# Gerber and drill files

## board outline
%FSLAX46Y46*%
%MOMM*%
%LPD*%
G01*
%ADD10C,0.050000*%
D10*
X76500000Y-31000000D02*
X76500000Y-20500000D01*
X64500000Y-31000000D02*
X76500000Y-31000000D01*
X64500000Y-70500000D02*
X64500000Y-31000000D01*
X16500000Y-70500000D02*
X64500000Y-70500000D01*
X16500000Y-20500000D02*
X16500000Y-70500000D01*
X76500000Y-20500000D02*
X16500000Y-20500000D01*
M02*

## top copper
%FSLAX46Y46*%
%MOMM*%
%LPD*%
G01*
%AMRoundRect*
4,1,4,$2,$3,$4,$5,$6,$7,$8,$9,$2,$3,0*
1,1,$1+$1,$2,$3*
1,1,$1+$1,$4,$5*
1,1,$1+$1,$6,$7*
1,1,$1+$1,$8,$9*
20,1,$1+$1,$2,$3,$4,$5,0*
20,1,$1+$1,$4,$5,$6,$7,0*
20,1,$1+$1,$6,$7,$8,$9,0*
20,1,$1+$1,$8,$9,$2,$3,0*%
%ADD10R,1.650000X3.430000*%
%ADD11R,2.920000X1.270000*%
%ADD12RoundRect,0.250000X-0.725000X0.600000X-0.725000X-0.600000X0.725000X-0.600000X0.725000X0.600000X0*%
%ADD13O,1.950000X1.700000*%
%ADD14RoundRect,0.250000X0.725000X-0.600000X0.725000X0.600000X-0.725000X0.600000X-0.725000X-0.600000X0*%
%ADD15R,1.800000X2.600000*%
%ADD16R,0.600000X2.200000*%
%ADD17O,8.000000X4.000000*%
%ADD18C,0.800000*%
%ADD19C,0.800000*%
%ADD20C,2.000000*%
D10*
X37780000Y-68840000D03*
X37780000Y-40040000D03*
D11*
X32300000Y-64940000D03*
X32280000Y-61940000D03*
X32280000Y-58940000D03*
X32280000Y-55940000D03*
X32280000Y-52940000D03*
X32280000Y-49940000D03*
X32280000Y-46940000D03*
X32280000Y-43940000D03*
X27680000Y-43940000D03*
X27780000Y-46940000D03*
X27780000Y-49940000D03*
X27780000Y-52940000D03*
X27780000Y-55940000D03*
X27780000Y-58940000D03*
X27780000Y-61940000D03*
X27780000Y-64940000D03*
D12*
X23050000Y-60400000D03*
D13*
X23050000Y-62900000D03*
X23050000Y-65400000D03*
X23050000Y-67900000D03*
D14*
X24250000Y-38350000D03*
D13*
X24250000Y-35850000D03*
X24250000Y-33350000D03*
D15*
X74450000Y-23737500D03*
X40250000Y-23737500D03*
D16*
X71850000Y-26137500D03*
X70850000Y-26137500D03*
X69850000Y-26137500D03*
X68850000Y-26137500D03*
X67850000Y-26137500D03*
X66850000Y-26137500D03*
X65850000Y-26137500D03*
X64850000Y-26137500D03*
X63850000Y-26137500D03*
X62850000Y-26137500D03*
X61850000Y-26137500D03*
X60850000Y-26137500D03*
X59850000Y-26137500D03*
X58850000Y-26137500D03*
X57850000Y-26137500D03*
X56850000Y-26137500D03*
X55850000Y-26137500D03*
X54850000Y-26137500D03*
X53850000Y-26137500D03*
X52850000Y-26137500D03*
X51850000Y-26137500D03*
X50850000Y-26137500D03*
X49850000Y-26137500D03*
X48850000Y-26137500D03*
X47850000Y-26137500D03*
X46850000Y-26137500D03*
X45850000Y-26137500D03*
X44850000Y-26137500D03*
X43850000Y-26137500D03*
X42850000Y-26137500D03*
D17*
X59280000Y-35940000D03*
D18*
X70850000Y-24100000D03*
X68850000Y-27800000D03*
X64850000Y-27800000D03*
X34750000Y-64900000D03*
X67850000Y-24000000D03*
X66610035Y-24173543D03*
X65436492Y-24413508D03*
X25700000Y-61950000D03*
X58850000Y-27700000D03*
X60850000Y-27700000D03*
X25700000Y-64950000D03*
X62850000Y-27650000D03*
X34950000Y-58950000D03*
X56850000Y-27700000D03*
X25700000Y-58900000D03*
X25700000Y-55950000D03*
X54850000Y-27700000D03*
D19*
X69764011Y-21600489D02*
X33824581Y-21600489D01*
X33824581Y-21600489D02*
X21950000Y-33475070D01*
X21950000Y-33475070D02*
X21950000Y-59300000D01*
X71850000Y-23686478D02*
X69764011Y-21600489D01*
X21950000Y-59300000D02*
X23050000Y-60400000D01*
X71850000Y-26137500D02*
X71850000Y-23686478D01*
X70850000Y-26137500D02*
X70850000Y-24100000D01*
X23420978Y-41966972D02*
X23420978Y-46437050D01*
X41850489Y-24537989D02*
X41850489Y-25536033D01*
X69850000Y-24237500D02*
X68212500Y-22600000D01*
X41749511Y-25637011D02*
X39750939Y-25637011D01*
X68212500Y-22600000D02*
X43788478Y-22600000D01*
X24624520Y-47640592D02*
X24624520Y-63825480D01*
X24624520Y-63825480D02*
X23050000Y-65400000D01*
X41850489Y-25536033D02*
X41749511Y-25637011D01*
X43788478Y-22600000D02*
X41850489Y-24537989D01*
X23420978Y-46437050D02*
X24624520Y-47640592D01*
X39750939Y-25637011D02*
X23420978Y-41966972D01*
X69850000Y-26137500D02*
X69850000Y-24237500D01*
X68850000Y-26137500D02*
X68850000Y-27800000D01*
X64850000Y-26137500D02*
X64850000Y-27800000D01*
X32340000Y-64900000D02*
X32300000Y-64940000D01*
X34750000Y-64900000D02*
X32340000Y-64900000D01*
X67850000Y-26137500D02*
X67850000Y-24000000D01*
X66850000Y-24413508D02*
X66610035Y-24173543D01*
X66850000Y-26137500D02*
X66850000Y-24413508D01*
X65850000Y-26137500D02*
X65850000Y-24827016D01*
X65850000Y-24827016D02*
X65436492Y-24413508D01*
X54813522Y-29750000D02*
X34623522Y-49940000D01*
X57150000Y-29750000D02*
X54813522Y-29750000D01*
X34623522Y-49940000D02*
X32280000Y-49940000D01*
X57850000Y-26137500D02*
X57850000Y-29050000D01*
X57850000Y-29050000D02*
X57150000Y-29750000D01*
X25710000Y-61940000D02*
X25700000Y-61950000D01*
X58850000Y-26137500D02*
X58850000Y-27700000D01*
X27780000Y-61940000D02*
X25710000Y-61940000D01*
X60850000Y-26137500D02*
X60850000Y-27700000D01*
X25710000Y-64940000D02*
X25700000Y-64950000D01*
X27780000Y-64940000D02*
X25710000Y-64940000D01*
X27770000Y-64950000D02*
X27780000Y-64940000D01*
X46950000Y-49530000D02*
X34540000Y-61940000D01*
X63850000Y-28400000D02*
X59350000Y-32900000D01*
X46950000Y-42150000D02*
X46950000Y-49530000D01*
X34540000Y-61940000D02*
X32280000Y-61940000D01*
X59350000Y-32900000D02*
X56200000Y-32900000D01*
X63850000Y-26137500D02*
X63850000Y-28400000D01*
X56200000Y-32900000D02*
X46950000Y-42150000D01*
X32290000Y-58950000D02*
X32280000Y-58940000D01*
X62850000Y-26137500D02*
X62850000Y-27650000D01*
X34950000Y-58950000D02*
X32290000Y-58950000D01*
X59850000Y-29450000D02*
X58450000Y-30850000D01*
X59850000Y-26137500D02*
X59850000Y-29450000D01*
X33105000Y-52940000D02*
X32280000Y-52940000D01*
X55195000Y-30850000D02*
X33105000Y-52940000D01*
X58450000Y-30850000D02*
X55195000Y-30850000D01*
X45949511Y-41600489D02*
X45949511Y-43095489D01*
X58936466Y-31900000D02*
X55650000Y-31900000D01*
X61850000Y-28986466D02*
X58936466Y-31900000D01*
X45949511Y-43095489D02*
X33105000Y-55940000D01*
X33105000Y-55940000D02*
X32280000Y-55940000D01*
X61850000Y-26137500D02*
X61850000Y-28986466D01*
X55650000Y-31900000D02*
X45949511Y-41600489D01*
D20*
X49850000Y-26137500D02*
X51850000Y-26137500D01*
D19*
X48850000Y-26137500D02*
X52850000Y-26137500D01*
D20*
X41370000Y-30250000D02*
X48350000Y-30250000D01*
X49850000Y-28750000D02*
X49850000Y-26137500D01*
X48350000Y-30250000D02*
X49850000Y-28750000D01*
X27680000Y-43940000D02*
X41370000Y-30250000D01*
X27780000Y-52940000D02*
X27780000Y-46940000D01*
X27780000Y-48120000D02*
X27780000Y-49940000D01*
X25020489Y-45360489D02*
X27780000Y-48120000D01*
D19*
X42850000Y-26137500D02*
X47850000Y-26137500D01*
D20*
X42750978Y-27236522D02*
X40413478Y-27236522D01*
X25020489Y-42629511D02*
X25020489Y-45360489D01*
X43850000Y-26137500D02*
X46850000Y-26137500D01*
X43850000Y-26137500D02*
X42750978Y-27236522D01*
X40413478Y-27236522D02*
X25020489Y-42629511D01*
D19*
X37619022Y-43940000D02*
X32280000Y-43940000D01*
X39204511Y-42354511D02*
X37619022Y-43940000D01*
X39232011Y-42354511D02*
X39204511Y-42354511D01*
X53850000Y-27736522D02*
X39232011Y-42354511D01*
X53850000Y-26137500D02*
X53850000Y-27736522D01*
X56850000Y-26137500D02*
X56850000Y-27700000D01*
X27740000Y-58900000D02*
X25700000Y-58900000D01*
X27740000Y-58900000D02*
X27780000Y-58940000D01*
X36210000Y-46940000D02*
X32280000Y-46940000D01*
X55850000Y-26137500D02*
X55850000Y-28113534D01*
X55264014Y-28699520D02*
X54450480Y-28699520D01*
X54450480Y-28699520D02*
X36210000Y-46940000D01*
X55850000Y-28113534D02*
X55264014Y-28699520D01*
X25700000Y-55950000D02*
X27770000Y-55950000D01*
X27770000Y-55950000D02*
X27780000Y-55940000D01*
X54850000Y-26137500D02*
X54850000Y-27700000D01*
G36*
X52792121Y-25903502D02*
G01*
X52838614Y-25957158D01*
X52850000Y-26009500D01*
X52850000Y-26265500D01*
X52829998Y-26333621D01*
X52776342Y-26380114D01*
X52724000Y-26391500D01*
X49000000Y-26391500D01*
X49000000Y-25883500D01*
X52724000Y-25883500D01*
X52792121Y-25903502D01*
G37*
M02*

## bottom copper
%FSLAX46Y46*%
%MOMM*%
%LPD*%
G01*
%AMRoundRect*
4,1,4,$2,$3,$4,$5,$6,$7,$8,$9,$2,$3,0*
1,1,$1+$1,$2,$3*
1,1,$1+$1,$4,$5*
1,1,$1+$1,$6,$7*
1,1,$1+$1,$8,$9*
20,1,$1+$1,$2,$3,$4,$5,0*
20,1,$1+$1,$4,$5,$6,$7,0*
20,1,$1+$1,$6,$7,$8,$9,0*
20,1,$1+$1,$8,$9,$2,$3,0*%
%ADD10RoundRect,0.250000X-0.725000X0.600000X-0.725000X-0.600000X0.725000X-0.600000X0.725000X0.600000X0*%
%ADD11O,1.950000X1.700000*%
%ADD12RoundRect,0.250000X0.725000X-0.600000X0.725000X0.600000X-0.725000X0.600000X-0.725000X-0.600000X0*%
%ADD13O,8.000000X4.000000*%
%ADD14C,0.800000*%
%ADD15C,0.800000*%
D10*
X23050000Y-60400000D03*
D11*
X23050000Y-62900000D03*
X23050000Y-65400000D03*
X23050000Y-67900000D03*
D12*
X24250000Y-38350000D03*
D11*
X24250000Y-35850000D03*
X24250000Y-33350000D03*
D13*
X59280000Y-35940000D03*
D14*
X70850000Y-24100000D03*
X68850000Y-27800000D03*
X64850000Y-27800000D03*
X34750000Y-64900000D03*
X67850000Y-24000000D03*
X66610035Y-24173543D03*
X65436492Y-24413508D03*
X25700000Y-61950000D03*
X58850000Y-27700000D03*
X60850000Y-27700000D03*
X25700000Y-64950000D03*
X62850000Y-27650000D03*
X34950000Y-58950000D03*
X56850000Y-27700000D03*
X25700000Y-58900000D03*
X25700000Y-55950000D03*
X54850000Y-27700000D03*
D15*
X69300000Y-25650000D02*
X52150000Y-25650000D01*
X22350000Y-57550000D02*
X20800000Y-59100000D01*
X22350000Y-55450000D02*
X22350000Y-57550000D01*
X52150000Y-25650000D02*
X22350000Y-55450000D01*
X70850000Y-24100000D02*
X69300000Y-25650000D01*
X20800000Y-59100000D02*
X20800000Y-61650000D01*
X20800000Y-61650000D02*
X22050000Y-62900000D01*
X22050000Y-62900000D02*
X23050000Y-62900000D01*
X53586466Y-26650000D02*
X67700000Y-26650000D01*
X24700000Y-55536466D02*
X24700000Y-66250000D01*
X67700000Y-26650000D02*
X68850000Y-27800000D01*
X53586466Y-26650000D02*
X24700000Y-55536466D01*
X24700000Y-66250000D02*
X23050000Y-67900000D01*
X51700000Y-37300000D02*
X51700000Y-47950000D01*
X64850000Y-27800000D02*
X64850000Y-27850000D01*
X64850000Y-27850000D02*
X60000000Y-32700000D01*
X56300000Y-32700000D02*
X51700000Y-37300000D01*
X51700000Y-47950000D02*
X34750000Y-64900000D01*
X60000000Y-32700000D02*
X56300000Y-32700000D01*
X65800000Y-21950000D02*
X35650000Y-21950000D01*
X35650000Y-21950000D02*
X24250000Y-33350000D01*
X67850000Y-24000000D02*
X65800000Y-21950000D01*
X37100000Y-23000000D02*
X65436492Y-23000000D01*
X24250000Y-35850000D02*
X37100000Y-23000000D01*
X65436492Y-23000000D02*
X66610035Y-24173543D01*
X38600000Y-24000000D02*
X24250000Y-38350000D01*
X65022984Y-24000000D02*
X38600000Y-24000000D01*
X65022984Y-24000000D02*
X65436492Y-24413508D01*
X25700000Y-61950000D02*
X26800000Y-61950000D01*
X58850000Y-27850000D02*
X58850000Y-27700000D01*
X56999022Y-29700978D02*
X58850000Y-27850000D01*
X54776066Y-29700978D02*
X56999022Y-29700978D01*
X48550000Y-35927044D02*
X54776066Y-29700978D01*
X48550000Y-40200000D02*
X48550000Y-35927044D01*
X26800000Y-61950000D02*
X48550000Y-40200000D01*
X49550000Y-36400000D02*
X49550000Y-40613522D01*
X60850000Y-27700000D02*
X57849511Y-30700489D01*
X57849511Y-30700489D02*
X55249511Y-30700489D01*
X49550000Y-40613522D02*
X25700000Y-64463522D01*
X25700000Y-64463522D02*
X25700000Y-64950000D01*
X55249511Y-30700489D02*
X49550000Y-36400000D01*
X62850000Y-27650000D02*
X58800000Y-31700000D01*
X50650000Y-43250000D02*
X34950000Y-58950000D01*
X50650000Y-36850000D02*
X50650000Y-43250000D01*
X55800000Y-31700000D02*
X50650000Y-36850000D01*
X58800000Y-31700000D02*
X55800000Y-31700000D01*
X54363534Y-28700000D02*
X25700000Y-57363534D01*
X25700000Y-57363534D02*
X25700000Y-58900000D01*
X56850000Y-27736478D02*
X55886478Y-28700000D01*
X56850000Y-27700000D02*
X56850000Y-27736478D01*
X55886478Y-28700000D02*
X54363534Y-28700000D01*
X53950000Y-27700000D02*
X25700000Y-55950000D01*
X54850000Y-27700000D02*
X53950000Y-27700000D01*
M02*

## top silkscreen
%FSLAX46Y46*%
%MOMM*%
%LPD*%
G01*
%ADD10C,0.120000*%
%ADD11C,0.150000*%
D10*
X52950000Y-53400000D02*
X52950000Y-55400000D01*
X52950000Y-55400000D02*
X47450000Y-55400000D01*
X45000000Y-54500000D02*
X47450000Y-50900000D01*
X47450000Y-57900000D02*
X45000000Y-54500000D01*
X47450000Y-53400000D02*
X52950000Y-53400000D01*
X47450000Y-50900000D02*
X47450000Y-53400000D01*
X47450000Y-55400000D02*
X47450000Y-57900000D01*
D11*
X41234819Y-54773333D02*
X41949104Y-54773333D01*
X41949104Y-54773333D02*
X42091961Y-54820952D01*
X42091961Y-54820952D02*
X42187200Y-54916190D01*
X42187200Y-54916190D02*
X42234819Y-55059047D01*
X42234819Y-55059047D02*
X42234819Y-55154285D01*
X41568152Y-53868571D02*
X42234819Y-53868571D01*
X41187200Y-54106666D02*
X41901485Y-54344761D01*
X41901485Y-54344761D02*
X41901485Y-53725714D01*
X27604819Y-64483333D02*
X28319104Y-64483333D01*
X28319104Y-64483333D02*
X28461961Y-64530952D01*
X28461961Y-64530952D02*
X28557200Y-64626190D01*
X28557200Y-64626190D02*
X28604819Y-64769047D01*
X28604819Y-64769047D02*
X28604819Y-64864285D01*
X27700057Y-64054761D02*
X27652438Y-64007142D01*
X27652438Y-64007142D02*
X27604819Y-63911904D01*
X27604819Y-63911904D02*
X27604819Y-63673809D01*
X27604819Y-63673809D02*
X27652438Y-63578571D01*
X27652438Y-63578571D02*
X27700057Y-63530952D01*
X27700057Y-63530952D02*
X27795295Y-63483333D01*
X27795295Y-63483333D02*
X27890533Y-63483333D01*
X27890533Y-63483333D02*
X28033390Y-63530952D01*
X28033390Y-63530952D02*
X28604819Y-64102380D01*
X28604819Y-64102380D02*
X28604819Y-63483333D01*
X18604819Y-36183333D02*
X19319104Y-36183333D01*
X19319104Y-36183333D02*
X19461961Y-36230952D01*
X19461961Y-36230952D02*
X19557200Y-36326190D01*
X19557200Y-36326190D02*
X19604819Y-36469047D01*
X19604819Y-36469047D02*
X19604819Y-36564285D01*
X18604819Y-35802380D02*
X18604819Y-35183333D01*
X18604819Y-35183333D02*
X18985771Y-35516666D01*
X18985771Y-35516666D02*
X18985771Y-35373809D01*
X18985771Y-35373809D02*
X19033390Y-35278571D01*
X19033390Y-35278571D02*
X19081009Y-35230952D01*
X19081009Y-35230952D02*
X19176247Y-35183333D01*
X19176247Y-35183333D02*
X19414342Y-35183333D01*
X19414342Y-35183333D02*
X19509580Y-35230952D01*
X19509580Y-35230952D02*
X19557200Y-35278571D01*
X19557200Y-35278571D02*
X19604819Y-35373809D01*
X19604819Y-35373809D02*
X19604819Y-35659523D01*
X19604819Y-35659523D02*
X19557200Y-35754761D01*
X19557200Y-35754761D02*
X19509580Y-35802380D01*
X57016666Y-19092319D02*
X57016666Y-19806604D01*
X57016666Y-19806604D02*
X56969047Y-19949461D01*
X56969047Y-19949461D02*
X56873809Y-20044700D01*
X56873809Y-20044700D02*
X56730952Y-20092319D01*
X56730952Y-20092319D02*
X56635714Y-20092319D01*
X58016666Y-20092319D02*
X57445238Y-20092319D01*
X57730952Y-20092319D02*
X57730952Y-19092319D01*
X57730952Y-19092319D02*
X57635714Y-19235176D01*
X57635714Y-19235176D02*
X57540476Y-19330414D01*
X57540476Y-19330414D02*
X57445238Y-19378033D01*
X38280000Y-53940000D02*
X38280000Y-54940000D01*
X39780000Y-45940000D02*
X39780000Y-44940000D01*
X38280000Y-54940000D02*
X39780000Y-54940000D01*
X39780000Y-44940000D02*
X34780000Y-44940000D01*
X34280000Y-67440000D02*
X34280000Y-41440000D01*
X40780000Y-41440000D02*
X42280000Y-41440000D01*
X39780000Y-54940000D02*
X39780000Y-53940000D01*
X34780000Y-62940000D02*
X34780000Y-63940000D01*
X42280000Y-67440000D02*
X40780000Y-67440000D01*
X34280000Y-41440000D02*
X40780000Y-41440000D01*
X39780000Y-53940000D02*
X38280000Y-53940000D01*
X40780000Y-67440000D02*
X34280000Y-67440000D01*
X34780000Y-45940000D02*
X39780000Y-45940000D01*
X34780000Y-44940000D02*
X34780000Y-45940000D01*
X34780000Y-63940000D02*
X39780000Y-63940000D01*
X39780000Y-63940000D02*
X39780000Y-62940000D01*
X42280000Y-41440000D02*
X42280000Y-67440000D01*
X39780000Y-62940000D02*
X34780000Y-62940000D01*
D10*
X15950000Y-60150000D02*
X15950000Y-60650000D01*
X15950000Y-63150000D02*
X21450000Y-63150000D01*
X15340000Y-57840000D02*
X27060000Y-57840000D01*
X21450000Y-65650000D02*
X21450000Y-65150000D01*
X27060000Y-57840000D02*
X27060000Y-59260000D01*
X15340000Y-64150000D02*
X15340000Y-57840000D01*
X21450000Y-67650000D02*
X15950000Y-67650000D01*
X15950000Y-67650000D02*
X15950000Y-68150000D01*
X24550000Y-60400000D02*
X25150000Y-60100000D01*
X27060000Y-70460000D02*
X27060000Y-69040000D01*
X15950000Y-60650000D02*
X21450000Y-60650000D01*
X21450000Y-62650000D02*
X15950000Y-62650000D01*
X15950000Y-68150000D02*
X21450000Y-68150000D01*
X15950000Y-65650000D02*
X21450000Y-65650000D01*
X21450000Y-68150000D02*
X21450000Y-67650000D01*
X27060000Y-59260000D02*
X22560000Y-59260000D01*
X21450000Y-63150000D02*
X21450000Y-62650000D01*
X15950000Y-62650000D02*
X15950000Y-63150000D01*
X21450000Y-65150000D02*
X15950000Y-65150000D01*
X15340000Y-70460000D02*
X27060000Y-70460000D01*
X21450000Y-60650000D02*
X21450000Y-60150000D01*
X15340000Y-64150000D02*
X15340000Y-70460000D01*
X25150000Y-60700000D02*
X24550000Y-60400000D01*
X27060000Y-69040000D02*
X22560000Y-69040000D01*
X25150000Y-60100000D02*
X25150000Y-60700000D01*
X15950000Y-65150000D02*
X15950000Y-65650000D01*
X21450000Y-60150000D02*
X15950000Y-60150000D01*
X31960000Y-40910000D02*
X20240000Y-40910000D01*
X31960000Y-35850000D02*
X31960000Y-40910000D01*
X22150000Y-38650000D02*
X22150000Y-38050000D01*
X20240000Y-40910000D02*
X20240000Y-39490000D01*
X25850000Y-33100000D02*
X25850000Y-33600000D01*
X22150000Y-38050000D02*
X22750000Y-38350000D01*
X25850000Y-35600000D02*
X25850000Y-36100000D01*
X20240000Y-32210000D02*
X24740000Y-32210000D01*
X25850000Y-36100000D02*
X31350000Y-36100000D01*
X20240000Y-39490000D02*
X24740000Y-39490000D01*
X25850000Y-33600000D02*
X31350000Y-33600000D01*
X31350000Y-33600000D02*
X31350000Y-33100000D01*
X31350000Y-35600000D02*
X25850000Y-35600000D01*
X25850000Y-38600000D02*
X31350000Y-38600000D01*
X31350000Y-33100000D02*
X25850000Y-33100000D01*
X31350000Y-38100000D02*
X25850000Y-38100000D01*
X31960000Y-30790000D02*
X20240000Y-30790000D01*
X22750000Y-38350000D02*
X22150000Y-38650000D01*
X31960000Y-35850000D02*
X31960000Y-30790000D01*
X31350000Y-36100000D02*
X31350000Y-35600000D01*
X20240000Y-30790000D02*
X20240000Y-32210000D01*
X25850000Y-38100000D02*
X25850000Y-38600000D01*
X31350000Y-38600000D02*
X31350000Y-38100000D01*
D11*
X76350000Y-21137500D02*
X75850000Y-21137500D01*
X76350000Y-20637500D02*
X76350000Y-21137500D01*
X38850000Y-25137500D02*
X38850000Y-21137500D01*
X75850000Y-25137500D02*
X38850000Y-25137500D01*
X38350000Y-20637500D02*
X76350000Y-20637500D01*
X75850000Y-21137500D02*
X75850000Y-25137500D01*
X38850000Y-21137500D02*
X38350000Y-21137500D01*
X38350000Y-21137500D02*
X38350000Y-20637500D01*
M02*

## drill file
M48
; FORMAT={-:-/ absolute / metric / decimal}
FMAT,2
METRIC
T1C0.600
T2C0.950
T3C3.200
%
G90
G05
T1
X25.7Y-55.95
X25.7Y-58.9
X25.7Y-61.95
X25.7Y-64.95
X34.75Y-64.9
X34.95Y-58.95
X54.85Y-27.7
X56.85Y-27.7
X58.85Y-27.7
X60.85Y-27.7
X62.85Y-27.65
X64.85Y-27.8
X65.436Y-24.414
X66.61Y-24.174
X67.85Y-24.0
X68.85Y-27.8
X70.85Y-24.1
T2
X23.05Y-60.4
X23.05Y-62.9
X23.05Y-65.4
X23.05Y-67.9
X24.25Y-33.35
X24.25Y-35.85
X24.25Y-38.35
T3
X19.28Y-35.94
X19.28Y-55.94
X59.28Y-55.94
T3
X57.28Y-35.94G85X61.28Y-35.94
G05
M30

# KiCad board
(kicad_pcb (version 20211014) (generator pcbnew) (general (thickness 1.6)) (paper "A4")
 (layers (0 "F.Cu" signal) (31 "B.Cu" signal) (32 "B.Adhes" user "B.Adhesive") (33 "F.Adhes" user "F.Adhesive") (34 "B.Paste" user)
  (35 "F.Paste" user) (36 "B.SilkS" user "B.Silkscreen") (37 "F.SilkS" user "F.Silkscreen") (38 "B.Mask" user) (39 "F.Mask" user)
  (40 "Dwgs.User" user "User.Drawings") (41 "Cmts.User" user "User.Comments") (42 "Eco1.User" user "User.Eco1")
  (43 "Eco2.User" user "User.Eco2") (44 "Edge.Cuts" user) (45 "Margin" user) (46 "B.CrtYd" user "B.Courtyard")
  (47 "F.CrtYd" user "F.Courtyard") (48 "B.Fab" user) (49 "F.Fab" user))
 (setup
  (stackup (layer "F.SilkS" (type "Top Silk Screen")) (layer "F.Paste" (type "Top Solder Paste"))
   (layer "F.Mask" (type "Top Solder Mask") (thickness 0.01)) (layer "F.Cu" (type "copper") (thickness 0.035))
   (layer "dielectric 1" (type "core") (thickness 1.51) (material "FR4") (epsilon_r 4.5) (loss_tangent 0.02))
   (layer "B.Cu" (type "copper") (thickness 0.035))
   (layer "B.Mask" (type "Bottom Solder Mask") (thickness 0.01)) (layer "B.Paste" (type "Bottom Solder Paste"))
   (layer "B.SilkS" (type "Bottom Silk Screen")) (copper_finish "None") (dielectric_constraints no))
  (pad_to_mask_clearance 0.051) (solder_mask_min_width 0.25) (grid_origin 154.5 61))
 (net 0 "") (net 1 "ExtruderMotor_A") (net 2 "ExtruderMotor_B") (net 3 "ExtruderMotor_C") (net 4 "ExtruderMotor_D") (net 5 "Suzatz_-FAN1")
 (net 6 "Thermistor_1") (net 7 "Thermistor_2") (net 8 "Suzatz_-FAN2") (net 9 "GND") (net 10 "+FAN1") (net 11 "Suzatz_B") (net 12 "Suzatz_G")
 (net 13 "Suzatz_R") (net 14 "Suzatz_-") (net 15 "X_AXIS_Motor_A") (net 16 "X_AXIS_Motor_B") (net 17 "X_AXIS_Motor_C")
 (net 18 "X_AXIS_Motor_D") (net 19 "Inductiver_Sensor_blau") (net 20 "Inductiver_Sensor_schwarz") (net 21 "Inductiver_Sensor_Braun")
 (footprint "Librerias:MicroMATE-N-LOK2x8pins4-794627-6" (layer "F.Cu") (at 37.78 54.44 90)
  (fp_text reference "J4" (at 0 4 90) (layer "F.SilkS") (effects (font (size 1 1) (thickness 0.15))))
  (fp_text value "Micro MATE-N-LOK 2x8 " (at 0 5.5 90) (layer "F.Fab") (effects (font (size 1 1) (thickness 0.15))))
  (fp_line (start 0.5 0.5) (end -0.5 0.5) (layer "F.SilkS") (width 0.15))
  (fp_line (start 8.5 2) (end 9.5 2) (layer "F.SilkS") (width 0.15))
  (fp_line (start -0.5 0.5) (end -0.5 2) (layer "F.SilkS") (width 0.15))
  (fp_line (start 9.5 2) (end 9.5 -3) (layer "F.SilkS") (width 0.15))
  (fp_line (start -13 -3.5) (end 13 -3.5) (layer "F.SilkS") (width 0.15))
  (fp_line (start 13 3) (end 13 4.5) (layer "F.SilkS") (width 0.15))
  (fp_line (start -0.5 2) (end 0.5 2) (layer "F.SilkS") (width 0.15))
  (fp_line (start -8.5 -3) (end -9.5 -3) (layer "F.SilkS") (width 0.15))
  (fp_line (start -13 4.5) (end -13 3) (layer "F.SilkS") (width 0.15))
  (fp_line (start 13 -3.5) (end 13 3) (layer "F.SilkS") (width 0.15))
  (fp_line (start 0.5 2) (end 0.5 0.5) (layer "F.SilkS") (width 0.15))
  (fp_line (start -13 3) (end -13 -3.5) (layer "F.SilkS") (width 0.15))
  (fp_line (start 8.5 -3) (end 8.5 2) (layer "F.SilkS") (width 0.15))
  (fp_line (start 9.5 -3) (end 8.5 -3) (layer "F.SilkS") (width 0.15))
  (fp_line (start -9.5 -3) (end -9.5 2) (layer "F.SilkS") (width 0.15))
  (fp_line (start -9.5 2) (end -8.5 2) (layer "F.SilkS") (width 0.15))
  (fp_line (start 13 4.5) (end -13 4.5) (layer "F.SilkS") (width 0.15))
  (fp_line (start -8.5 2) (end -8.5 -3) (layer "F.SilkS") (width 0.15))
  (pad "0" smd rect locked (at -14.4 0 90) (size 3.43 1.65) (layers "F.Cu" "F.Paste" "F.Mask"))
  (pad "0" smd rect locked (at 14.4 0 90) (size 3.43 1.65) (layers "F.Cu" "F.Paste" "F.Mask"))
  (pad "1" smd rect locked (at -10.5 -5.48 270) (size 1.27 2.92) (layers "F.Cu" "F.Paste" "F.Mask") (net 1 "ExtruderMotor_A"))
  (pad "2" smd rect locked (at -7.5 -5.5 270) (size 1.27 2.92) (layers "F.Cu" "F.Paste" "F.Mask") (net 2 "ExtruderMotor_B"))
  (pad "3" smd rect locked (at -4.5 -5.5 270) (size 1.27 2.92) (layers "F.Cu" "F.Paste" "F.Mask") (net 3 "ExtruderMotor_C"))
  (pad "4" smd rect locked (at -1.5 -5.5 270) (size 1.27 2.92) (layers "F.Cu" "F.Paste" "F.Mask") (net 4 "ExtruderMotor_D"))
  (pad "5" smd rect locked (at 1.5 -5.5 270) (size 1.27 2.92) (layers "F.Cu" "F.Paste" "F.Mask") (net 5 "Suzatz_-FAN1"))
  (pad "6" smd rect locked (at 4.5 -5.5 270) (size 1.27 2.92) (layers "F.Cu" "F.Paste" "F.Mask") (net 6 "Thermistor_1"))
  (pad "7" smd rect locked (at 7.5 -5.5 270) (size 1.27 2.92) (layers "F.Cu" "F.Paste" "F.Mask") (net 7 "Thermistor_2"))
  (pad "8" smd rect locked (at 10.5 -5.5 270) (size 1.27 2.92) (layers "F.Cu" "F.Paste" "F.Mask") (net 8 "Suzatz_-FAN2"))
  (pad "9" smd rect locked (at 10.5 -10.1 270) (size 1.27 2.92) (layers "F.Cu" "F.Paste" "F.Mask") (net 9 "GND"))
  (pad "10" smd rect locked (at 7.5 -10 270) (size 1.27 2.92) (layers "F.Cu" "F.Paste" "F.Mask") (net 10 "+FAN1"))
  (pad "11" smd rect locked (at 4.5 -10 270) (size 1.27 2.92) (layers "F.Cu" "F.Paste" "F.Mask") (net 10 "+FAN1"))
  (pad "12" smd rect locked (at 1.5 -10 270) (size 1.27 2.92) (layers "F.Cu" "F.Paste" "F.Mask") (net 10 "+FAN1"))
  (pad "13" smd rect locked (at -1.5 -10 270) (size 1.27 2.92) (layers "F.Cu" "F.Paste" "F.Mask") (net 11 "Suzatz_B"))
  (pad "14" smd rect locked (at -4.5 -10 270) (size 1.27 2.92) (layers "F.Cu" "F.Paste" "F.Mask") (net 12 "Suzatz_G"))
  (pad "15" smd rect locked (at -7.5 -10 270) (size 1.27 2.92) (layers "F.Cu" "F.Paste" "F.Mask") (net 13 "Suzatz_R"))
  (pad "16" smd rect locked (at -10.5 -10 270) (size 1.27 2.92) (layers "F.Cu" "F.Paste" "F.Mask") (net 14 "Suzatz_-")))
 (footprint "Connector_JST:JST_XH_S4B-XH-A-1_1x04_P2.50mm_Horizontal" (layer "F.Cu") (at 23.05 60.4 -90)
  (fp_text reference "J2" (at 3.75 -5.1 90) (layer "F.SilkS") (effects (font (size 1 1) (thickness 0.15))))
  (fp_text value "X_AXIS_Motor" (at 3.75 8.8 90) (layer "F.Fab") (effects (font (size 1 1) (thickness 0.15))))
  (fp_line (start -0.25 7.1) (end 0.25 7.1) (layer "F.SilkS") (width 0.12))
  (fp_line (start 2.75 7.1) (end 2.75 1.6) (layer "F.SilkS") (width 0.12))
  (fp_line (start -2.56 7.71) (end -2.56 -4.01) (layer "F.SilkS") (width 0.12))
  (fp_line (start 5.25 1.6) (end 4.75 1.6) (layer "F.SilkS") (width 0.12))
  (fp_line (start -2.56 -4.01) (end -1.14 -4.01) (layer "F.SilkS") (width 0.12))
  (fp_line (start 3.75 7.71) (end -2.56 7.71) (layer "F.SilkS") (width 0.12))
  (fp_line (start 7.25 1.6) (end 7.25 7.1) (layer "F.SilkS") (width 0.12))
  (fp_line (start 7.25 7.1) (end 7.75 7.1) (layer "F.SilkS") (width 0.12))
  (fp_line (start 0 -1.5) (end -0.3 -2.1) (layer "F.SilkS") (width 0.12))
  (fp_line (start 10.06 -4.01) (end 8.64 -4.01) (layer "F.SilkS") (width 0.12))
  (fp_line (start 0.25 7.1) (end 0.25 1.6) (layer "F.SilkS") (width 0.12))
  (fp_line (start 2.25 1.6) (end 2.25 7.1) (layer "F.SilkS") (width 0.12))
  (fp_line (start 7.75 7.1) (end 7.75 1.6) (layer "F.SilkS") (width 0.12))
  (fp_line (start 5.25 7.1) (end 5.25 1.6) (layer "F.SilkS") (width 0.12))
  (fp_line (start 7.75 1.6) (end 7.25 1.6) (layer "F.SilkS") (width 0.12))
  (fp_line (start -1.14 -4.01) (end -1.14 0.49) (layer "F.SilkS") (width 0.12))
  (fp_line (start 2.75 1.6) (end 2.25 1.6) (layer "F.SilkS") (width 0.12))
  (fp_line (start 2.25 7.1) (end 2.75 7.1) (layer "F.SilkS") (width 0.12))
  (fp_line (start 4.75 1.6) (end 4.75 7.1) (layer "F.SilkS") (width 0.12))
  (fp_line (start 10.06 7.71) (end 10.06 -4.01) (layer "F.SilkS") (width 0.12))
  (fp_line (start 0.25 1.6) (end -0.25 1.6) (layer "F.SilkS") (width 0.12))
  (fp_line (start 3.75 7.71) (end 10.06 7.71) (layer "F.SilkS") (width 0.12))
  (fp_line (start 0.3 -2.1) (end 0 -1.5) (layer "F.SilkS") (width 0.12))
  (fp_line (start 8.64 -4.01) (end 8.64 0.49) (layer "F.SilkS") (width 0.12))
  (fp_line (start -0.3 -2.1) (end 0.3 -2.1) (layer "F.SilkS") (width 0.12))
  (fp_line (start 4.75 7.1) (end 5.25 7.1) (layer "F.SilkS") (width 0.12))
  (fp_line (start -0.25 1.6) (end -0.25 7.1) (layer "F.SilkS") (width 0.12))
  (pad "1" thru_hole roundrect locked (at 0 0 270) (size 1.7 1.95) (drill 0.95) (layers *.Cu *.Mask) (roundrect_rratio 0.147059)
   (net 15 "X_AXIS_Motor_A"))
  (pad "2" thru_hole oval locked (at 2.5 0 270) (size 1.7 1.95) (drill 0.95) (layers *.Cu *.Mask) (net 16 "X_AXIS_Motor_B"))
  (pad "3" thru_hole oval locked (at 5 0 270) (size 1.7 1.95) (drill 0.95) (layers *.Cu *.Mask) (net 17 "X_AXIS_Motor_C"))
  (pad "4" thru_hole oval locked (at 7.5 0 270) (size 1.7 1.95) (drill 0.95) (layers *.Cu *.Mask) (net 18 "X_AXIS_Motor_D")))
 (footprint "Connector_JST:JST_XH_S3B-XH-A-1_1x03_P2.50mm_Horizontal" (layer "F.Cu") (at 24.25 38.35 90)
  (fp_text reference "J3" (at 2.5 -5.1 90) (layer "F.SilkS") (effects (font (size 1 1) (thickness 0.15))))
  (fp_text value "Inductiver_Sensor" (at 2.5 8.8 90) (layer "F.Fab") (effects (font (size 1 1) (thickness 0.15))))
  (fp_line (start -2.56 7.71) (end -2.56 -4.01) (layer "F.SilkS") (width 0.12))
  (fp_line (start 2.5 7.71) (end -2.56 7.71) (layer "F.SilkS") (width 0.12))
  (fp_line (start -0.3 -2.1) (end 0.3 -2.1) (layer "F.SilkS") (width 0.12))
  (fp_line (start -2.56 -4.01) (end -1.14 -4.01) (layer "F.SilkS") (width 0.12))
  (fp_line (start 5.25 1.6) (end 4.75 1.6) (layer "F.SilkS") (width 0.12))
  (fp_line (start 0.3 -2.1) (end 0 -1.5) (layer "F.SilkS") (width 0.12))
  (fp_line (start 2.75 1.6) (end 2.25 1.6) (layer "F.SilkS") (width 0.12))
  (fp_line (start 6.14 -4.01) (end 6.14 0.49) (layer "F.SilkS") (width 0.12))
  (fp_line (start 2.25 1.6) (end 2.25 7.1) (layer "F.SilkS") (width 0.12))
  (fp_line (start -1.14 -4.01) (end -1.14 0.49) (layer "F.SilkS") (width 0.12))
  (fp_line (start 4.75 1.6) (end 4.75 7.1) (layer "F.SilkS") (width 0.12))
  (fp_line (start 4.75 7.1) (end 5.25 7.1) (layer "F.SilkS") (width 0.12))
  (fp_line (start 2.75 7.1) (end 2.75 1.6) (layer "F.SilkS") (width 0.12))
  (fp_line (start -0.25 1.6) (end -0.25 7.1) (layer "F.SilkS") (width 0.12))
  (fp_line (start 5.25 7.1) (end 5.25 1.6) (layer "F.SilkS") (width 0.12))
  (fp_line (start 0.25 7.1) (end 0.25 1.6) (layer "F.SilkS") (width 0.12))
  (fp_line (start 7.56 7.71) (end 7.56 -4.01) (layer "F.SilkS") (width 0.12))
  (fp_line (start 0 -1.5) (end -0.3 -2.1) (layer "F.SilkS") (width 0.12))
  (fp_line (start 2.5 7.71) (end 7.56 7.71) (layer "F.SilkS") (width 0.12))
  (fp_line (start 2.25 7.1) (end 2.75 7.1) (layer "F.SilkS") (width 0.12))
  (fp_line (start 7.56 -4.01) (end 6.14 -4.01) (layer "F.SilkS") (width 0.12))
  (fp_line (start 0.25 1.6) (end -0.25 1.6) (layer "F.SilkS") (width 0.12))
  (fp_line (start -0.25 7.1) (end 0.25 7.1) (layer "F.SilkS") (width 0.12))
  (pad "1" thru_hole roundrect locked (at 0 0 90) (size 1.7 1.95) (drill 0.95) (layers *.Cu *.Mask) (roundrect_rratio 0.147059)
   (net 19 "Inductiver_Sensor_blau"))
  (pad "2" thru_hole oval locked (at 2.5 0 90) (size 1.7 1.95) (drill 0.95) (layers *.Cu *.Mask) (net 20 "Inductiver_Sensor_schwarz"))
  (pad "3" thru_hole oval locked (at 5 0 90) (size 1.7 1.95) (drill 0.95) (layers *.Cu *.Mask) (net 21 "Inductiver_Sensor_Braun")))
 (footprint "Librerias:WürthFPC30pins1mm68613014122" (layer "F.Cu") (at 57.35 25.1375 180)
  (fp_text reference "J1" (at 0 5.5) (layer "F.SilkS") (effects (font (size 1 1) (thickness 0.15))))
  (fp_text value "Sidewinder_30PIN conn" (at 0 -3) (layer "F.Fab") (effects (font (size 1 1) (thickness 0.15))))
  (fp_line (start -19 4) (end -18.5 4) (layer "F.SilkS") (width 0.15))
  (fp_line (start -19 4.5) (end -19 4) (layer "F.SilkS") (width 0.15))
  (fp_line (start 18.5 0) (end 18.5 4) (layer "F.SilkS") (width 0.15))
  (fp_line (start -18.5 0) (end 18.5 0) (layer "F.SilkS") (width 0.15))
  (fp_line (start 19 4.5) (end -19 4.5) (layer "F.SilkS") (width 0.15))
  (fp_line (start -18.5 4) (end -18.5 0) (layer "F.SilkS") (width 0.15))
  (fp_line (start 18.5 4) (end 19 4) (layer "F.SilkS") (width 0.15))
  (fp_line (start 19 4) (end 19 4.5) (layer "F.SilkS") (width 0.15))
  (pad "0" smd rect locked (at -17.1 1.4 180) (size 1.8 2.6) (layers "F.Cu" "F.Paste" "F.Mask"))
  (pad "0" smd rect locked (at 17.1 1.4 180) (size 1.8 2.6) (layers "F.Cu" "F.Paste" "F.Mask"))
  (pad "1" smd rect locked (at -14.5 -1 180) (size 0.6 2.2) (layers "F.Cu" "F.Paste" "F.Mask") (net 15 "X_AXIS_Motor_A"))
  (pad "2" smd rect locked (at -13.5 -1 180) (size 0.6 2.2) (layers "F.Cu" "F.Paste" "F.Mask") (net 16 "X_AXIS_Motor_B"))
  (pad "3" smd rect locked (at -12.5 -1 180) (size 0.6 2.2) (layers "F.Cu" "F.Paste" "F.Mask") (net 17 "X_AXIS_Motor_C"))
  (pad "4" smd rect locked (at -11.5 -1 180) (size 0.6 2.2) (layers "F.Cu" "F.Paste" "F.Mask") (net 18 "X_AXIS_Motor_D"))
  (pad "5" smd rect locked (at -10.5 -1 180) (size 0.6 2.2) (layers "F.Cu" "F.Paste" "F.Mask") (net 21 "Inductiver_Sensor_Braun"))
  (pad "6" smd rect locked (at -9.5 -1 180) (size 0.6 2.2) (layers "F.Cu" "F.Paste" "F.Mask") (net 20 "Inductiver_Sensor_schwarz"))
  (pad "7" smd rect locked (at -8.5 -1 180) (size 0.6 2.2) (layers "F.Cu" "F.Paste" "F.Mask") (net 19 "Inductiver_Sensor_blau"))
  (pad "8" smd rect locked (at -7.5 -1 180) (size 0.6 2.2) (layers "F.Cu" "F.Paste" "F.Mask") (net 1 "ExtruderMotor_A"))
  (pad "9" smd rect locked (at -6.5 -1 180) (size 0.6 2.2) (layers "F.Cu" "F.Paste" "F.Mask") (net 2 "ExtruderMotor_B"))
  (pad "10" smd rect locked (at -5.5 -1 180) (size 0.6 2.2) (layers "F.Cu" "F.Paste" "F.Mask") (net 3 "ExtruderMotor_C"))
  (pad "11" smd rect locked (at -4.5 -1 180) (size 0.6 2.2) (layers "F.Cu" "F.Paste" "F.Mask") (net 4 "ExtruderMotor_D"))
  (pad "12" smd rect locked (at -3.5 -1 180) (size 0.6 2.2) (layers "F.Cu" "F.Paste" "F.Mask") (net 14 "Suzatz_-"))
  (pad "13" smd rect locked (at -2.5 -1 180) (size 0.6 2.2) (layers "F.Cu" "F.Paste" "F.Mask") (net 5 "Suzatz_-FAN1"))
  (pad "14" smd rect locked (at -1.5 -1 180) (size 0.6 2.2) (layers "F.Cu" "F.Paste" "F.Mask") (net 13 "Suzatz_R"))
  (pad "15" smd rect locked (at -0.5 -1 180) (size 0.6 2.2) (layers "F.Cu" "F.Paste" "F.Mask") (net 6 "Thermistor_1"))
  (pad "16" smd rect locked (at 0.5 -1 180) (size 0.6 2.2) (layers "F.Cu" "F.Paste" "F.Mask") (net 12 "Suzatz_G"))
  (pad "17" smd rect locked (at 1.5 -1 180) (size 0.6 2.2) (layers "F.Cu" "F.Paste" "F.Mask") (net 7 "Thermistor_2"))
  (pad "18" smd rect locked (at 2.5 -1 180) (size 0.6 2.2) (layers "F.Cu" "F.Paste" "F.Mask") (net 11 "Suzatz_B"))
  (pad "19" smd rect locked (at 3.5 -1 180) (size 0.6 2.2) (layers "F.Cu" "F.Paste" "F.Mask") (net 8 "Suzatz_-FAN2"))
  (pad "20" smd rect locked (at 4.5 -1 180) (size 0.6 2.2) (layers "F.Cu" "F.Paste" "F.Mask") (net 9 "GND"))
  (pad "21" smd rect locked (at 5.5 -1 180) (size 0.6 2.2) (layers "F.Cu" "F.Paste" "F.Mask") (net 9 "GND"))
  (pad "22" smd rect locked (at 6.5 -1 180) (size 0.6 2.2) (layers "F.Cu" "F.Paste" "F.Mask") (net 9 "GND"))
  (pad "23" smd rect locked (at 7.5 -1 180) (size 0.6 2.2) (layers "F.Cu" "F.Paste" "F.Mask") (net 9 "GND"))
  (pad "24" smd rect locked (at 8.5 -1 180) (size 0.6 2.2) (layers "F.Cu" "F.Paste" "F.Mask") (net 9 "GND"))
  (pad "25" smd rect locked (at 9.5 -1 180) (size 0.6 2.2) (layers "F.Cu" "F.Paste" "F.Mask") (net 10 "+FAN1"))
  (pad "26" smd rect locked (at 10.5 -1 180) (size 0.6 2.2) (layers "F.Cu" "F.Paste" "F.Mask") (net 10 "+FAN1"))
  (pad "27" smd rect locked (at 11.5 -1 180) (size 0.6 2.2) (layers "F.Cu" "F.Paste" "F.Mask") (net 10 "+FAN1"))
  (pad "28" smd rect locked (at 12.5 -1 180) (size 0.6 2.2) (layers "F.Cu" "F.Paste" "F.Mask") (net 10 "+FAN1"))
  (pad "29" smd rect locked (at 13.5 -1 180) (size 0.6 2.2) (layers "F.Cu" "F.Paste" "F.Mask") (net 10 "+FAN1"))
  (pad "30" smd rect locked (at 14.5 -1 180) (size 0.6 2.2) (layers "F.Cu" "F.Paste" "F.Mask") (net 10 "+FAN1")))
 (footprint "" (layer "F.Cu") (at 8.05 35.4)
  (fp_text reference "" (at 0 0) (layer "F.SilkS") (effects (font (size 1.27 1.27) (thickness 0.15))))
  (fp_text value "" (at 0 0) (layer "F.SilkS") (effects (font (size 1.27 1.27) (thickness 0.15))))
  (pad "" np_thru_hole circle (at 11.23 0.54) (size 3.2 3.2) (drill 3.2) (layers F&B.Cu *.Mask)))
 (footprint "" (layer "F.Cu") (at 14.35 56)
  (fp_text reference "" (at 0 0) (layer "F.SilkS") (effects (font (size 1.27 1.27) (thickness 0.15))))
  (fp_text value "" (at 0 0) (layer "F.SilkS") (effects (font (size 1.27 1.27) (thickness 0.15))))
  (pad "" np_thru_hole circle locked (at 4.93 -0.06) (size 3.2 3.2) (drill 3.2) (layers F&B.Cu *.Mask)))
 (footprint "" (layer "F.Cu") (at 71.5 37.6)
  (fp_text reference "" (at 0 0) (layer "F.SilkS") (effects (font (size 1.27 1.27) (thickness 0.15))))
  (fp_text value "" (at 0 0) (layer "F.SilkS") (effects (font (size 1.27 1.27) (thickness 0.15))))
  (pad "" np_thru_hole oval (at -12.22 -1.66) (size 8 4) (drill oval 7.2 3.2) (layers F&B.Cu *.Mask)))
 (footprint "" (layer "F.Cu") (at 63.25 54.95)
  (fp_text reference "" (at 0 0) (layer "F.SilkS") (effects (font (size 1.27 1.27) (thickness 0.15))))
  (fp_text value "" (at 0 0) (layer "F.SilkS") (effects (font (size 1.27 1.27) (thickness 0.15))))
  (pad "" np_thru_hole circle (at -3.97 0.99) (size 3.2 3.2) (drill 3.2) (layers F&B.Cu *.Mask)))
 (gr_line (start 52.95 53.4) (end 52.95 55.4) (layer "F.SilkS") (width 0.12))
 (gr_line (start 52.95 55.4) (end 47.45 55.4) (layer "F.SilkS") (width 0.12))
 (gr_line (start 45 54.5) (end 47.45 50.9) (layer "F.SilkS") (width 0.12))
 (gr_line (start 47.45 57.9) (end 45 54.5) (layer "F.SilkS") (width 0.12))
 (gr_line (start 47.45 53.4) (end 52.95 53.4) (layer "F.SilkS") (width 0.12))
 (gr_line (start 47.45 50.9) (end 47.45 53.4) (layer "F.SilkS") (width 0.12))
 (gr_line (start 47.45 55.4) (end 47.45 57.9) (layer "F.SilkS") (width 0.12))
 (gr_line (start 76.5 31) (end 76.5 20.5) (layer "Edge.Cuts") (width 0.05))
 (gr_line (start 64.5 31) (end 76.5 31) (layer "Edge.Cuts") (width 0.05))
 (gr_line (start 64.5 70.5) (end 64.5 31) (layer "Edge.Cuts") (width 0.05))
 (gr_line (start 16.5 70.5) (end 64.5 70.5) (layer "Edge.Cuts") (width 0.05))
 (gr_line (start 16.5 20.5) (end 16.5 70.5) (layer "Edge.Cuts") (width 0.05))
 (gr_line (start 76.5 20.5) (end 16.5 20.5) (layer "Edge.Cuts") (width 0.05))
 (segment (start 69.764011 21.600489) (end 33.824581 21.600489) (width 0.8) (layer "F.Cu") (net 15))
 (segment (start 33.824581 21.600489) (end 21.95 33.47507) (width 0.8) (layer "F.Cu") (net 15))
 (segment locked (start 21.95 33.47507) (end 21.95 59.3) (width 0.8) (layer "F.Cu") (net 15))
 (segment (start 71.85 23.686478) (end 69.764011 21.600489) (width 0.8) (layer "F.Cu") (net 15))
 (segment (start 21.95 59.3) (end 23.05 60.4) (width 0.8) (layer "F.Cu") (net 15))
 (segment (start 71.85 26.1375) (end 71.85 23.686478) (width 0.8) (layer "F.Cu") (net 15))
 (segment (start 70.85 26.1375) (end 70.85 24.1) (width 0.8) (layer "F.Cu") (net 16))
 (via (at 70.85 24.1) (size 0.8) (drill 0.6) (layers "F.Cu" "B.Cu") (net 16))
 (segment (start 69.3 25.65) (end 52.15 25.65) (width 0.8) (layer "B.Cu") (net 16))
 (segment (start 22.35 57.55) (end 20.8 59.1) (width 0.8) (layer "B.Cu") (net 16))
 (segment (start 22.35 55.45) (end 22.35 57.55) (width 0.8) (layer "B.Cu") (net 16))
 (segment (start 52.15 25.65) (end 22.35 55.45) (width 0.8) (layer "B.Cu") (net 16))
 (segment (start 70.85 24.1) (end 69.3 25.65) (width 0.8) (layer "B.Cu") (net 16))
 (segment (start 20.8 59.1) (end 20.8 61.65) (width 0.8) (layer "B.Cu") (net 16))
 (segment (start 20.8 61.65) (end 22.05 62.9) (width 0.8) (layer "B.Cu") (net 16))
 (segment (start 22.05 62.9) (end 23.05 62.9) (width 0.8) (layer "B.Cu") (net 16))
 (segment (start 23.420978 41.966972) (end 23.420978 46.43705) (width 0.8) (layer "F.Cu") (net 17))
 (segment (start 41.850489 24.537989) (end 41.850489 25.536033) (width 0.8) (layer "F.Cu") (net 17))
 (segment (start 69.85 24.2375) (end 68.2125 22.6) (width 0.8) (layer "F.Cu") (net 17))
 (segment (start 41.749511 25.637011) (end 39.750939 25.637011) (width 0.8) (layer "F.Cu") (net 17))
 (segment (start 68.2125 22.6) (end 43.788478 22.6) (width 0.8) (layer "F.Cu") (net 17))
 (segment (start 24.62452 47.640592) (end 24.62452 63.82548) (width 0.8) (layer "F.Cu") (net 17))
 (segment (start 24.62452 63.82548) (end 23.05 65.4) (width 0.8) (layer "F.Cu") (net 17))
 (segment (start 41.850489 25.536033) (end 41.749511 25.637011) (width 0.8) (layer "F.Cu") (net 17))
 (segment (start 43.788478 22.6) (end 41.850489 24.537989) (width 0.8) (layer "F.Cu") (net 17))
 (segment (start 23.420978 46.43705) (end 24.62452 47.640592) (width 0.8) (layer "F.Cu") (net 17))
 (segment (start 39.750939 25.637011) (end 23.420978 41.966972) (width 0.8) (layer "F.Cu") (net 17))
 (segment (start 69.85 26.1375) (end 69.85 24.2375) (width 0.8) (layer "F.Cu") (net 17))
 (segment (start 68.85 26.1375) (end 68.85 27.8) (width 0.8) (layer "F.Cu") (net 18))
 (via (at 68.85 27.8) (size 0.8) (drill 0.6) (layers "F.Cu" "B.Cu") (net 18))
 (segment locked (start 53.586466 26.65) (end 67.7 26.65) (width 0.8) (layer "B.Cu") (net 18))
 (segment (start 24.7 55.536466) (end 24.7 66.25) (width 0.8) (layer "B.Cu") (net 18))
 (segment (start 67.7 26.65) (end 68.85 27.8) (width 0.8) (layer "B.Cu") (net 18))
 (segment (start 53.586466 26.65) (end 24.7 55.536466) (width 0.8) (layer "B.Cu") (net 18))
 (segment (start 24.7 66.25) (end 23.05 67.9) (width 0.8) (layer "B.Cu") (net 18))
 (segment (start 64.85 26.1375) (end 64.85 27.8) (width 0.8) (layer "F.Cu") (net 1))
 (segment (start 32.34 64.9) (end 32.3 64.94) (width 0.8) (layer "F.Cu") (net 1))
 (segment (start 34.75 64.9) (end 32.34 64.9) (width 0.8) (layer "F.Cu") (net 1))
 (via locked (at 64.85 27.8) (size 0.8) (drill 0.6) (layers "F.Cu" "B.Cu") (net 1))
 (via (at 34.75 64.9) (size 0.8) (drill 0.6) (layers "F.Cu" "B.Cu") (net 1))
 (segment (start 51.7 37.3) (end 51.7 47.95) (width 0.8) (layer "B.Cu") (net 1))
 (segment (start 64.85 27.8) (end 64.85 27.85) (width 0.8) (layer "B.Cu") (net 1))
 (segment (start 64.85 27.85) (end 60 32.7) (width 0.8) (layer "B.Cu") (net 1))
 (segment (start 56.3 32.7) (end 51.7 37.3) (width 0.8) (layer "B.Cu") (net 1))
 (segment (start 51.7 47.95) (end 34.75 64.9) (width 0.8) (layer "B.Cu") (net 1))
 (segment (start 60 32.7) (end 56.3 32.7) (width 0.8) (layer "B.Cu") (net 1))
 (segment (start 67.85 26.1375) (end 67.85 24) (width 0.8) (layer "F.Cu") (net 21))
 (via (at 67.85 24) (size 0.8) (drill 0.6) (layers "F.Cu" "B.Cu") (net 21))
 (segment (start 65.8 21.95) (end 35.65 21.95) (width 0.8) (layer "B.Cu") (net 21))
 (segment (start 35.65 21.95) (end 24.25 33.35) (width 0.8) (layer "B.Cu") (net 21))
 (segment (start 67.85 24) (end 65.8 21.95) (width 0.8) (layer "B.Cu") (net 21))
 (segment (start 66.85 24.413508) (end 66.610035 24.173543) (width 0.8) (layer "F.Cu") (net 20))
 (segment (start 66.85 26.1375) (end 66.85 24.413508) (width 0.8) (layer "F.Cu") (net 20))
 (via (at 66.610035 24.173543) (size 0.8) (drill 0.6) (layers "F.Cu" "B.Cu") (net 20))
 (segment (start 37.1 23) (end 65.436492 23) (width 0.8) (layer "B.Cu") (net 20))
 (segment (start 24.25 35.85) (end 37.1 23) (width 0.8) (layer "B.Cu") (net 20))
 (segment (start 65.436492 23) (end 66.610035 24.173543) (width 0.8) (layer "B.Cu") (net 20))
 (segment (start 65.85 26.1375) (end 65.85 24.827016) (width 0.8) (layer "F.Cu") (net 19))
 (segment (start 65.85 24.827016) (end 65.436492 24.413508) (width 0.8) (layer "F.Cu") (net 19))
 (via (at 65.436492 24.413508) (size 0.8) (drill 0.6) (layers "F.Cu" "B.Cu") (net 19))
 (segment (start 38.6 24) (end 24.25 38.35) (width 0.8) (layer "B.Cu") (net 19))
 (segment (start 65.022984 24) (end 38.6 24) (width 0.8) (layer "B.Cu") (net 19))
 (segment (start 65.022984 24) (end 65.436492 24.413508) (width 0.8) (layer "B.Cu") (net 19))
 (segment (start 54.813522 29.75) (end 34.623522 49.94) (width 0.8) (layer "F.Cu") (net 6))
 (segment (start 57.15 29.75) (end 54.813522 29.75) (width 0.8) (layer "F.Cu") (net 6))
 (segment (start 34.623522 49.94) (end 32.28 49.94) (width 0.8) (layer "F.Cu") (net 6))
 (segment (start 57.85 26.1375) (end 57.85 29.05) (width 0.8) (layer "F.Cu") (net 6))
 (segment (start 57.85 29.05) (end 57.15 29.75) (width 0.8) (layer "F.Cu") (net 6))
 (segment (start 25.71 61.94) (end 25.7 61.95) (width 0.8) (layer "F.Cu") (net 13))
 (segment (start 58.85 26.1375) (end 58.85 27.7) (width 0.8) (layer "F.Cu") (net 13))
 (segment (start 27.78 61.94) (end 25.71 61.94) (width 0.8) (layer "F.Cu") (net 13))
 (via locked (at 25.7 61.95) (size 0.8) (drill 0.6) (layers "F.Cu" "B.Cu") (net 13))
 (via locked (at 58.85 27.7) (size 0.8) (drill 0.6) (layers "F.Cu" "B.Cu") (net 13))
 (segment (start 25.7 61.95) (end 26.8 61.95) (width 0.8) (layer "B.Cu") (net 13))
 (segment (start 58.85 27.85) (end 58.85 27.7) (width 0.8) (layer "B.Cu") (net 13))
 (segment (start 56.999022 29.700978) (end 58.85 27.85) (width 0.8) (layer "B.Cu") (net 13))
 (segment (start 54.776066 29.700978) (end 56.999022 29.700978) (width 0.8) (layer "B.Cu") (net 13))
 (segment (start 48.55 35.927044) (end 54.776066 29.700978) (width 0.8) (layer "B.Cu") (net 13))
 (segment (start 48.55 40.2) (end 48.55 35.927044) (width 0.8) (layer "B.Cu") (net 13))
 (segment (start 26.8 61.95) (end 48.55 40.2) (width 0.8) (layer "B.Cu") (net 13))
 (segment (start 60.85 26.1375) (end 60.85 27.7) (width 0.8) (layer "F.Cu") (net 14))
 (segment (start 25.71 64.94) (end 25.7 64.95) (width 0.8) (layer "F.Cu") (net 14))
 (segment (start 27.78 64.94) (end 25.71 64.94) (width 0.8) (layer "F.Cu") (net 14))
 (segment (start 27.77 64.95) (end 27.78 64.94) (width 0.8) (layer "F.Cu") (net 14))
 (via locked (at 60.85 27.7) (size 0.8) (drill 0.6) (layers "F.Cu" "B.Cu") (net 14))
 (via locked (at 25.7 64.95) (size 0.8) (drill 0.6) (layers "F.Cu" "B.Cu") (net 14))
 (segment (start 49.55 36.4) (end 49.55 40.613522) (width 0.8) (layer "B.Cu") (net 14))
 (segment (start 60.85 27.7) (end 57.849511 30.700489) (width 0.8) (layer "B.Cu") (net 14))
 (segment (start 57.849511 30.700489) (end 55.249511 30.700489) (width 0.8) (layer "B.Cu") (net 14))
 (segment (start 49.55 40.613522) (end 25.7 64.463522) (width 0.8) (layer "B.Cu") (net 14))
 (segment (start 25.7 64.463522) (end 25.7 64.95) (width 0.8) (layer "B.Cu") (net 14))
 (segment (start 55.249511 30.700489) (end 49.55 36.4) (width 0.8) (layer "B.Cu") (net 14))
 (segment (start 46.95 49.53) (end 34.54 61.94) (width 0.8) (layer "F.Cu") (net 2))
 (segment locked (start 63.85 28.4) (end 59.35 32.9) (width 0.8) (layer "F.Cu") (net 2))
 (segment (start 46.95 42.15) (end 46.95 49.53) (width 0.8) (layer "F.Cu") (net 2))
 (segment (start 34.54 61.94) (end 32.28 61.94) (width 0.8) (layer "F.Cu") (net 2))
 (segment locked (start 59.35 32.9) (end 56.2 32.9) (width 0.8) (layer "F.Cu") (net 2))
 (segment (start 63.85 26.1375) (end 63.85 28.4) (width 0.8) (layer "F.Cu") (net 2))
 (segment locked (start 56.2 32.9) (end 46.95 42.15) (width 0.8) (layer "F.Cu") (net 2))
 (segment (start 32.29 58.95) (end 32.28 58.94) (width 0.8) (layer "F.Cu") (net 3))
 (segment (start 62.85 26.1375) (end 62.85 27.65) (width 0.8) (layer "F.Cu") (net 3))
 (segment (start 34.95 58.95) (end 32.29 58.95) (width 0.8) (layer "F.Cu") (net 3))
 (via locked (at 62.85 27.65) (size 0.8) (drill 0.6) (layers "F.Cu" "B.Cu") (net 3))
 (via (at 34.95 58.95) (size 0.8) (drill 0.6) (layers "F.Cu" "B.Cu") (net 3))
 (segment (start 62.85 27.65) (end 58.8 31.7) (width 0.8) (layer "B.Cu") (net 3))
 (segment (start 50.65 43.25) (end 34.95 58.95) (width 0.8) (layer "B.Cu") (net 3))
 (segment (start 50.65 36.85) (end 50.65 43.25) (width 0.8) (layer "B.Cu") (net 3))
 (segment (start 55.8 31.7) (end 50.65 36.85) (width 0.8) (layer "B.Cu") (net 3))
 (segment (start 58.8 31.7) (end 55.8 31.7) (width 0.8) (layer "B.Cu") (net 3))
 (segment (start 59.85 29.45) (end 58.45 30.85) (width 0.8) (layer "F.Cu") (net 5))
 (segment (start 59.85 26.1375) (end 59.85 29.45) (width 0.8) (layer "F.Cu") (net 5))
 (segment (start 33.105 52.94) (end 32.28 52.94) (width 0.8) (layer "F.Cu") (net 5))
 (segment (start 55.195 30.85) (end 33.105 52.94) (width 0.8) (layer "F.Cu") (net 5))
 (segment (start 58.45 30.85) (end 55.195 30.85) (width 0.8) (layer "F.Cu") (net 5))
 (segment (start 45.949511 41.600489) (end 45.949511 43.095489) (width 0.8) (layer "F.Cu") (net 4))
 (segment (start 58.936466 31.9) (end 55.65 31.9) (width 0.8) (layer "F.Cu") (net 4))
 (segment (start 61.85 28.986466) (end 58.936466 31.9) (width 0.8) (layer "F.Cu") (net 4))
 (segment (start 45.949511 43.095489) (end 33.105 55.94) (width 0.8) (layer "F.Cu") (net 4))
 (segment (start 33.105 55.94) (end 32.28 55.94) (width 0.8) (layer "F.Cu") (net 4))
 (segment (start 61.85 26.1375) (end 61.85 28.986466) (width 0.8) (layer "F.Cu") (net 4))
 (segment (start 55.65 31.9) (end 45.949511 41.600489) (width 0.8) (layer "F.Cu") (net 4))
 (segment (start 49.85 26.1375) (end 51.85 26.1375) (width 2) (layer "F.Cu") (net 9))
 (segment (start 48.85 26.1375) (end 52.85 26.1375) (width 0.8) (layer "F.Cu") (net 9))
 (segment (start 41.37 30.25) (end 48.35 30.25) (width 2) (layer "F.Cu") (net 9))
 (segment (start 49.85 28.75) (end 49.85 26.1375) (width 2) (layer "F.Cu") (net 9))
 (segment (start 48.35 30.25) (end 49.85 28.75) (width 2) (layer "F.Cu") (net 9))
 (segment (start 27.68 43.94) (end 41.37 30.25) (width 2) (layer "F.Cu") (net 9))
 (segment (start 27.78 52.94) (end 27.78 46.94) (width 2) (layer "F.Cu") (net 10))
 (segment (start 27.78 48.12) (end 27.78 49.94) (width 2) (layer "F.Cu") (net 10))
 (segment (start 25.020489 45.360489) (end 27.78 48.12) (width 2) (layer "F.Cu") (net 10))
 (segment (start 42.85 26.1375) (end 47.85 26.1375) (width 0.8) (layer "F.Cu") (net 10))
 (segment (start 42.750978 27.236522) (end 40.413478 27.236522) (width 2) (layer "F.Cu") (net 10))
 (segment (start 25.020489 42.629511) (end 25.020489 45.360489) (width 2) (layer "F.Cu") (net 10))
 (segment (start 43.85 26.1375) (end 46.85 26.1375) (width 2) (layer "F.Cu") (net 10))
 (segment (start 43.85 26.1375) (end 42.750978 27.236522) (width 2) (layer "F.Cu") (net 10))
 (segment (start 40.413478 27.236522) (end 25.020489 42.629511) (width 2) (layer "F.Cu") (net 10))
 (segment (start 37.619022 43.94) (end 32.28 43.94) (width 0.8) (layer "F.Cu") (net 8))
 (segment (start 39.204511 42.354511) (end 37.619022 43.94) (width 0.8) (layer "F.Cu") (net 8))
 (segment (start 39.232011 42.354511) (end 39.204511 42.354511) (width 0.8) (layer "F.Cu") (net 8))
 (segment (start 53.85 27.736522) (end 39.232011 42.354511) (width 0.8) (layer "F.Cu") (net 8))
 (segment (start 53.85 26.1375) (end 53.85 27.736522) (width 0.8) (layer "F.Cu") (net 8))
 (segment (start 56.85 26.1375) (end 56.85 27.7) (width 0.8) (layer "F.Cu") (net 12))
 (segment (start 27.74 58.9) (end 25.7 58.9) (width 0.8) (layer "F.Cu") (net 12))
 (segment (start 27.74 58.9) (end 27.78 58.94) (width 0.8) (layer "F.Cu") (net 12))
 (via locked (at 56.85 27.7) (size 0.8) (drill 0.6) (layers "F.Cu" "B.Cu") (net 12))
 (via locked (at 25.7 58.9) (size 0.8) (drill 0.6) (layers "F.Cu" "B.Cu") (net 12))
 (segment (start 54.363534 28.7) (end 25.7 57.363534) (width 0.8) (layer "B.Cu") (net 12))
 (segment (start 25.7 57.363534) (end 25.7 58.9) (width 0.8) (layer "B.Cu") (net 12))
 (segment (start 56.85 27.736478) (end 55.886478 28.7) (width 0.8) (layer "B.Cu") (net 12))
 (segment (start 56.85 27.7) (end 56.85 27.736478) (width 0.8) (layer "B.Cu") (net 12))
 (segment (start 55.886478 28.7) (end 54.363534 28.7) (width 0.8) (layer "B.Cu") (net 12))
 (segment (start 36.21 46.94) (end 32.28 46.94) (width 0.8) (layer "F.Cu") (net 7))
 (segment (start 55.85 26.1375) (end 55.85 28.113534) (width 0.8) (layer "F.Cu") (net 7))
 (segment (start 55.264014 28.69952) (end 54.45048 28.69952) (width 0.8) (layer "F.Cu") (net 7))
 (segment (start 54.45048 28.69952) (end 36.21 46.94) (width 0.8) (layer "F.Cu") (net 7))
 (segment (start 55.85 28.113534) (end 55.264014 28.69952) (width 0.8) (layer "F.Cu") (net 7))
 (segment (start 25.7 55.95) (end 27.77 55.95) (width 0.8) (layer "F.Cu") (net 11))
 (segment (start 27.77 55.95) (end 27.78 55.94) (width 0.8) (layer "F.Cu") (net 11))
 (segment (start 54.85 26.1375) (end 54.85 27.7) (width 0.8) (layer "F.Cu") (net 11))
 (via locked (at 25.7 55.95) (size 0.8) (drill 0.6) (layers "F.Cu" "B.Cu") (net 11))
 (via locked (at 54.85 27.7) (size 0.8) (drill 0.6) (layers "F.Cu" "B.Cu") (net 11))
 (segment (start 53.95 27.7) (end 25.7 55.95) (width 0.8) (layer "B.Cu") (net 11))
 (segment (start 54.85 27.7) (end 53.95 27.7) (width 0.8) (layer "B.Cu") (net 11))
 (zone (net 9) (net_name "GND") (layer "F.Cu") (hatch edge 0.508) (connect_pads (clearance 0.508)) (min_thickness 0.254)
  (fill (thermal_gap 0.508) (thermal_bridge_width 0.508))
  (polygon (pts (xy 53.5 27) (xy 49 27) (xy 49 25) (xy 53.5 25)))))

